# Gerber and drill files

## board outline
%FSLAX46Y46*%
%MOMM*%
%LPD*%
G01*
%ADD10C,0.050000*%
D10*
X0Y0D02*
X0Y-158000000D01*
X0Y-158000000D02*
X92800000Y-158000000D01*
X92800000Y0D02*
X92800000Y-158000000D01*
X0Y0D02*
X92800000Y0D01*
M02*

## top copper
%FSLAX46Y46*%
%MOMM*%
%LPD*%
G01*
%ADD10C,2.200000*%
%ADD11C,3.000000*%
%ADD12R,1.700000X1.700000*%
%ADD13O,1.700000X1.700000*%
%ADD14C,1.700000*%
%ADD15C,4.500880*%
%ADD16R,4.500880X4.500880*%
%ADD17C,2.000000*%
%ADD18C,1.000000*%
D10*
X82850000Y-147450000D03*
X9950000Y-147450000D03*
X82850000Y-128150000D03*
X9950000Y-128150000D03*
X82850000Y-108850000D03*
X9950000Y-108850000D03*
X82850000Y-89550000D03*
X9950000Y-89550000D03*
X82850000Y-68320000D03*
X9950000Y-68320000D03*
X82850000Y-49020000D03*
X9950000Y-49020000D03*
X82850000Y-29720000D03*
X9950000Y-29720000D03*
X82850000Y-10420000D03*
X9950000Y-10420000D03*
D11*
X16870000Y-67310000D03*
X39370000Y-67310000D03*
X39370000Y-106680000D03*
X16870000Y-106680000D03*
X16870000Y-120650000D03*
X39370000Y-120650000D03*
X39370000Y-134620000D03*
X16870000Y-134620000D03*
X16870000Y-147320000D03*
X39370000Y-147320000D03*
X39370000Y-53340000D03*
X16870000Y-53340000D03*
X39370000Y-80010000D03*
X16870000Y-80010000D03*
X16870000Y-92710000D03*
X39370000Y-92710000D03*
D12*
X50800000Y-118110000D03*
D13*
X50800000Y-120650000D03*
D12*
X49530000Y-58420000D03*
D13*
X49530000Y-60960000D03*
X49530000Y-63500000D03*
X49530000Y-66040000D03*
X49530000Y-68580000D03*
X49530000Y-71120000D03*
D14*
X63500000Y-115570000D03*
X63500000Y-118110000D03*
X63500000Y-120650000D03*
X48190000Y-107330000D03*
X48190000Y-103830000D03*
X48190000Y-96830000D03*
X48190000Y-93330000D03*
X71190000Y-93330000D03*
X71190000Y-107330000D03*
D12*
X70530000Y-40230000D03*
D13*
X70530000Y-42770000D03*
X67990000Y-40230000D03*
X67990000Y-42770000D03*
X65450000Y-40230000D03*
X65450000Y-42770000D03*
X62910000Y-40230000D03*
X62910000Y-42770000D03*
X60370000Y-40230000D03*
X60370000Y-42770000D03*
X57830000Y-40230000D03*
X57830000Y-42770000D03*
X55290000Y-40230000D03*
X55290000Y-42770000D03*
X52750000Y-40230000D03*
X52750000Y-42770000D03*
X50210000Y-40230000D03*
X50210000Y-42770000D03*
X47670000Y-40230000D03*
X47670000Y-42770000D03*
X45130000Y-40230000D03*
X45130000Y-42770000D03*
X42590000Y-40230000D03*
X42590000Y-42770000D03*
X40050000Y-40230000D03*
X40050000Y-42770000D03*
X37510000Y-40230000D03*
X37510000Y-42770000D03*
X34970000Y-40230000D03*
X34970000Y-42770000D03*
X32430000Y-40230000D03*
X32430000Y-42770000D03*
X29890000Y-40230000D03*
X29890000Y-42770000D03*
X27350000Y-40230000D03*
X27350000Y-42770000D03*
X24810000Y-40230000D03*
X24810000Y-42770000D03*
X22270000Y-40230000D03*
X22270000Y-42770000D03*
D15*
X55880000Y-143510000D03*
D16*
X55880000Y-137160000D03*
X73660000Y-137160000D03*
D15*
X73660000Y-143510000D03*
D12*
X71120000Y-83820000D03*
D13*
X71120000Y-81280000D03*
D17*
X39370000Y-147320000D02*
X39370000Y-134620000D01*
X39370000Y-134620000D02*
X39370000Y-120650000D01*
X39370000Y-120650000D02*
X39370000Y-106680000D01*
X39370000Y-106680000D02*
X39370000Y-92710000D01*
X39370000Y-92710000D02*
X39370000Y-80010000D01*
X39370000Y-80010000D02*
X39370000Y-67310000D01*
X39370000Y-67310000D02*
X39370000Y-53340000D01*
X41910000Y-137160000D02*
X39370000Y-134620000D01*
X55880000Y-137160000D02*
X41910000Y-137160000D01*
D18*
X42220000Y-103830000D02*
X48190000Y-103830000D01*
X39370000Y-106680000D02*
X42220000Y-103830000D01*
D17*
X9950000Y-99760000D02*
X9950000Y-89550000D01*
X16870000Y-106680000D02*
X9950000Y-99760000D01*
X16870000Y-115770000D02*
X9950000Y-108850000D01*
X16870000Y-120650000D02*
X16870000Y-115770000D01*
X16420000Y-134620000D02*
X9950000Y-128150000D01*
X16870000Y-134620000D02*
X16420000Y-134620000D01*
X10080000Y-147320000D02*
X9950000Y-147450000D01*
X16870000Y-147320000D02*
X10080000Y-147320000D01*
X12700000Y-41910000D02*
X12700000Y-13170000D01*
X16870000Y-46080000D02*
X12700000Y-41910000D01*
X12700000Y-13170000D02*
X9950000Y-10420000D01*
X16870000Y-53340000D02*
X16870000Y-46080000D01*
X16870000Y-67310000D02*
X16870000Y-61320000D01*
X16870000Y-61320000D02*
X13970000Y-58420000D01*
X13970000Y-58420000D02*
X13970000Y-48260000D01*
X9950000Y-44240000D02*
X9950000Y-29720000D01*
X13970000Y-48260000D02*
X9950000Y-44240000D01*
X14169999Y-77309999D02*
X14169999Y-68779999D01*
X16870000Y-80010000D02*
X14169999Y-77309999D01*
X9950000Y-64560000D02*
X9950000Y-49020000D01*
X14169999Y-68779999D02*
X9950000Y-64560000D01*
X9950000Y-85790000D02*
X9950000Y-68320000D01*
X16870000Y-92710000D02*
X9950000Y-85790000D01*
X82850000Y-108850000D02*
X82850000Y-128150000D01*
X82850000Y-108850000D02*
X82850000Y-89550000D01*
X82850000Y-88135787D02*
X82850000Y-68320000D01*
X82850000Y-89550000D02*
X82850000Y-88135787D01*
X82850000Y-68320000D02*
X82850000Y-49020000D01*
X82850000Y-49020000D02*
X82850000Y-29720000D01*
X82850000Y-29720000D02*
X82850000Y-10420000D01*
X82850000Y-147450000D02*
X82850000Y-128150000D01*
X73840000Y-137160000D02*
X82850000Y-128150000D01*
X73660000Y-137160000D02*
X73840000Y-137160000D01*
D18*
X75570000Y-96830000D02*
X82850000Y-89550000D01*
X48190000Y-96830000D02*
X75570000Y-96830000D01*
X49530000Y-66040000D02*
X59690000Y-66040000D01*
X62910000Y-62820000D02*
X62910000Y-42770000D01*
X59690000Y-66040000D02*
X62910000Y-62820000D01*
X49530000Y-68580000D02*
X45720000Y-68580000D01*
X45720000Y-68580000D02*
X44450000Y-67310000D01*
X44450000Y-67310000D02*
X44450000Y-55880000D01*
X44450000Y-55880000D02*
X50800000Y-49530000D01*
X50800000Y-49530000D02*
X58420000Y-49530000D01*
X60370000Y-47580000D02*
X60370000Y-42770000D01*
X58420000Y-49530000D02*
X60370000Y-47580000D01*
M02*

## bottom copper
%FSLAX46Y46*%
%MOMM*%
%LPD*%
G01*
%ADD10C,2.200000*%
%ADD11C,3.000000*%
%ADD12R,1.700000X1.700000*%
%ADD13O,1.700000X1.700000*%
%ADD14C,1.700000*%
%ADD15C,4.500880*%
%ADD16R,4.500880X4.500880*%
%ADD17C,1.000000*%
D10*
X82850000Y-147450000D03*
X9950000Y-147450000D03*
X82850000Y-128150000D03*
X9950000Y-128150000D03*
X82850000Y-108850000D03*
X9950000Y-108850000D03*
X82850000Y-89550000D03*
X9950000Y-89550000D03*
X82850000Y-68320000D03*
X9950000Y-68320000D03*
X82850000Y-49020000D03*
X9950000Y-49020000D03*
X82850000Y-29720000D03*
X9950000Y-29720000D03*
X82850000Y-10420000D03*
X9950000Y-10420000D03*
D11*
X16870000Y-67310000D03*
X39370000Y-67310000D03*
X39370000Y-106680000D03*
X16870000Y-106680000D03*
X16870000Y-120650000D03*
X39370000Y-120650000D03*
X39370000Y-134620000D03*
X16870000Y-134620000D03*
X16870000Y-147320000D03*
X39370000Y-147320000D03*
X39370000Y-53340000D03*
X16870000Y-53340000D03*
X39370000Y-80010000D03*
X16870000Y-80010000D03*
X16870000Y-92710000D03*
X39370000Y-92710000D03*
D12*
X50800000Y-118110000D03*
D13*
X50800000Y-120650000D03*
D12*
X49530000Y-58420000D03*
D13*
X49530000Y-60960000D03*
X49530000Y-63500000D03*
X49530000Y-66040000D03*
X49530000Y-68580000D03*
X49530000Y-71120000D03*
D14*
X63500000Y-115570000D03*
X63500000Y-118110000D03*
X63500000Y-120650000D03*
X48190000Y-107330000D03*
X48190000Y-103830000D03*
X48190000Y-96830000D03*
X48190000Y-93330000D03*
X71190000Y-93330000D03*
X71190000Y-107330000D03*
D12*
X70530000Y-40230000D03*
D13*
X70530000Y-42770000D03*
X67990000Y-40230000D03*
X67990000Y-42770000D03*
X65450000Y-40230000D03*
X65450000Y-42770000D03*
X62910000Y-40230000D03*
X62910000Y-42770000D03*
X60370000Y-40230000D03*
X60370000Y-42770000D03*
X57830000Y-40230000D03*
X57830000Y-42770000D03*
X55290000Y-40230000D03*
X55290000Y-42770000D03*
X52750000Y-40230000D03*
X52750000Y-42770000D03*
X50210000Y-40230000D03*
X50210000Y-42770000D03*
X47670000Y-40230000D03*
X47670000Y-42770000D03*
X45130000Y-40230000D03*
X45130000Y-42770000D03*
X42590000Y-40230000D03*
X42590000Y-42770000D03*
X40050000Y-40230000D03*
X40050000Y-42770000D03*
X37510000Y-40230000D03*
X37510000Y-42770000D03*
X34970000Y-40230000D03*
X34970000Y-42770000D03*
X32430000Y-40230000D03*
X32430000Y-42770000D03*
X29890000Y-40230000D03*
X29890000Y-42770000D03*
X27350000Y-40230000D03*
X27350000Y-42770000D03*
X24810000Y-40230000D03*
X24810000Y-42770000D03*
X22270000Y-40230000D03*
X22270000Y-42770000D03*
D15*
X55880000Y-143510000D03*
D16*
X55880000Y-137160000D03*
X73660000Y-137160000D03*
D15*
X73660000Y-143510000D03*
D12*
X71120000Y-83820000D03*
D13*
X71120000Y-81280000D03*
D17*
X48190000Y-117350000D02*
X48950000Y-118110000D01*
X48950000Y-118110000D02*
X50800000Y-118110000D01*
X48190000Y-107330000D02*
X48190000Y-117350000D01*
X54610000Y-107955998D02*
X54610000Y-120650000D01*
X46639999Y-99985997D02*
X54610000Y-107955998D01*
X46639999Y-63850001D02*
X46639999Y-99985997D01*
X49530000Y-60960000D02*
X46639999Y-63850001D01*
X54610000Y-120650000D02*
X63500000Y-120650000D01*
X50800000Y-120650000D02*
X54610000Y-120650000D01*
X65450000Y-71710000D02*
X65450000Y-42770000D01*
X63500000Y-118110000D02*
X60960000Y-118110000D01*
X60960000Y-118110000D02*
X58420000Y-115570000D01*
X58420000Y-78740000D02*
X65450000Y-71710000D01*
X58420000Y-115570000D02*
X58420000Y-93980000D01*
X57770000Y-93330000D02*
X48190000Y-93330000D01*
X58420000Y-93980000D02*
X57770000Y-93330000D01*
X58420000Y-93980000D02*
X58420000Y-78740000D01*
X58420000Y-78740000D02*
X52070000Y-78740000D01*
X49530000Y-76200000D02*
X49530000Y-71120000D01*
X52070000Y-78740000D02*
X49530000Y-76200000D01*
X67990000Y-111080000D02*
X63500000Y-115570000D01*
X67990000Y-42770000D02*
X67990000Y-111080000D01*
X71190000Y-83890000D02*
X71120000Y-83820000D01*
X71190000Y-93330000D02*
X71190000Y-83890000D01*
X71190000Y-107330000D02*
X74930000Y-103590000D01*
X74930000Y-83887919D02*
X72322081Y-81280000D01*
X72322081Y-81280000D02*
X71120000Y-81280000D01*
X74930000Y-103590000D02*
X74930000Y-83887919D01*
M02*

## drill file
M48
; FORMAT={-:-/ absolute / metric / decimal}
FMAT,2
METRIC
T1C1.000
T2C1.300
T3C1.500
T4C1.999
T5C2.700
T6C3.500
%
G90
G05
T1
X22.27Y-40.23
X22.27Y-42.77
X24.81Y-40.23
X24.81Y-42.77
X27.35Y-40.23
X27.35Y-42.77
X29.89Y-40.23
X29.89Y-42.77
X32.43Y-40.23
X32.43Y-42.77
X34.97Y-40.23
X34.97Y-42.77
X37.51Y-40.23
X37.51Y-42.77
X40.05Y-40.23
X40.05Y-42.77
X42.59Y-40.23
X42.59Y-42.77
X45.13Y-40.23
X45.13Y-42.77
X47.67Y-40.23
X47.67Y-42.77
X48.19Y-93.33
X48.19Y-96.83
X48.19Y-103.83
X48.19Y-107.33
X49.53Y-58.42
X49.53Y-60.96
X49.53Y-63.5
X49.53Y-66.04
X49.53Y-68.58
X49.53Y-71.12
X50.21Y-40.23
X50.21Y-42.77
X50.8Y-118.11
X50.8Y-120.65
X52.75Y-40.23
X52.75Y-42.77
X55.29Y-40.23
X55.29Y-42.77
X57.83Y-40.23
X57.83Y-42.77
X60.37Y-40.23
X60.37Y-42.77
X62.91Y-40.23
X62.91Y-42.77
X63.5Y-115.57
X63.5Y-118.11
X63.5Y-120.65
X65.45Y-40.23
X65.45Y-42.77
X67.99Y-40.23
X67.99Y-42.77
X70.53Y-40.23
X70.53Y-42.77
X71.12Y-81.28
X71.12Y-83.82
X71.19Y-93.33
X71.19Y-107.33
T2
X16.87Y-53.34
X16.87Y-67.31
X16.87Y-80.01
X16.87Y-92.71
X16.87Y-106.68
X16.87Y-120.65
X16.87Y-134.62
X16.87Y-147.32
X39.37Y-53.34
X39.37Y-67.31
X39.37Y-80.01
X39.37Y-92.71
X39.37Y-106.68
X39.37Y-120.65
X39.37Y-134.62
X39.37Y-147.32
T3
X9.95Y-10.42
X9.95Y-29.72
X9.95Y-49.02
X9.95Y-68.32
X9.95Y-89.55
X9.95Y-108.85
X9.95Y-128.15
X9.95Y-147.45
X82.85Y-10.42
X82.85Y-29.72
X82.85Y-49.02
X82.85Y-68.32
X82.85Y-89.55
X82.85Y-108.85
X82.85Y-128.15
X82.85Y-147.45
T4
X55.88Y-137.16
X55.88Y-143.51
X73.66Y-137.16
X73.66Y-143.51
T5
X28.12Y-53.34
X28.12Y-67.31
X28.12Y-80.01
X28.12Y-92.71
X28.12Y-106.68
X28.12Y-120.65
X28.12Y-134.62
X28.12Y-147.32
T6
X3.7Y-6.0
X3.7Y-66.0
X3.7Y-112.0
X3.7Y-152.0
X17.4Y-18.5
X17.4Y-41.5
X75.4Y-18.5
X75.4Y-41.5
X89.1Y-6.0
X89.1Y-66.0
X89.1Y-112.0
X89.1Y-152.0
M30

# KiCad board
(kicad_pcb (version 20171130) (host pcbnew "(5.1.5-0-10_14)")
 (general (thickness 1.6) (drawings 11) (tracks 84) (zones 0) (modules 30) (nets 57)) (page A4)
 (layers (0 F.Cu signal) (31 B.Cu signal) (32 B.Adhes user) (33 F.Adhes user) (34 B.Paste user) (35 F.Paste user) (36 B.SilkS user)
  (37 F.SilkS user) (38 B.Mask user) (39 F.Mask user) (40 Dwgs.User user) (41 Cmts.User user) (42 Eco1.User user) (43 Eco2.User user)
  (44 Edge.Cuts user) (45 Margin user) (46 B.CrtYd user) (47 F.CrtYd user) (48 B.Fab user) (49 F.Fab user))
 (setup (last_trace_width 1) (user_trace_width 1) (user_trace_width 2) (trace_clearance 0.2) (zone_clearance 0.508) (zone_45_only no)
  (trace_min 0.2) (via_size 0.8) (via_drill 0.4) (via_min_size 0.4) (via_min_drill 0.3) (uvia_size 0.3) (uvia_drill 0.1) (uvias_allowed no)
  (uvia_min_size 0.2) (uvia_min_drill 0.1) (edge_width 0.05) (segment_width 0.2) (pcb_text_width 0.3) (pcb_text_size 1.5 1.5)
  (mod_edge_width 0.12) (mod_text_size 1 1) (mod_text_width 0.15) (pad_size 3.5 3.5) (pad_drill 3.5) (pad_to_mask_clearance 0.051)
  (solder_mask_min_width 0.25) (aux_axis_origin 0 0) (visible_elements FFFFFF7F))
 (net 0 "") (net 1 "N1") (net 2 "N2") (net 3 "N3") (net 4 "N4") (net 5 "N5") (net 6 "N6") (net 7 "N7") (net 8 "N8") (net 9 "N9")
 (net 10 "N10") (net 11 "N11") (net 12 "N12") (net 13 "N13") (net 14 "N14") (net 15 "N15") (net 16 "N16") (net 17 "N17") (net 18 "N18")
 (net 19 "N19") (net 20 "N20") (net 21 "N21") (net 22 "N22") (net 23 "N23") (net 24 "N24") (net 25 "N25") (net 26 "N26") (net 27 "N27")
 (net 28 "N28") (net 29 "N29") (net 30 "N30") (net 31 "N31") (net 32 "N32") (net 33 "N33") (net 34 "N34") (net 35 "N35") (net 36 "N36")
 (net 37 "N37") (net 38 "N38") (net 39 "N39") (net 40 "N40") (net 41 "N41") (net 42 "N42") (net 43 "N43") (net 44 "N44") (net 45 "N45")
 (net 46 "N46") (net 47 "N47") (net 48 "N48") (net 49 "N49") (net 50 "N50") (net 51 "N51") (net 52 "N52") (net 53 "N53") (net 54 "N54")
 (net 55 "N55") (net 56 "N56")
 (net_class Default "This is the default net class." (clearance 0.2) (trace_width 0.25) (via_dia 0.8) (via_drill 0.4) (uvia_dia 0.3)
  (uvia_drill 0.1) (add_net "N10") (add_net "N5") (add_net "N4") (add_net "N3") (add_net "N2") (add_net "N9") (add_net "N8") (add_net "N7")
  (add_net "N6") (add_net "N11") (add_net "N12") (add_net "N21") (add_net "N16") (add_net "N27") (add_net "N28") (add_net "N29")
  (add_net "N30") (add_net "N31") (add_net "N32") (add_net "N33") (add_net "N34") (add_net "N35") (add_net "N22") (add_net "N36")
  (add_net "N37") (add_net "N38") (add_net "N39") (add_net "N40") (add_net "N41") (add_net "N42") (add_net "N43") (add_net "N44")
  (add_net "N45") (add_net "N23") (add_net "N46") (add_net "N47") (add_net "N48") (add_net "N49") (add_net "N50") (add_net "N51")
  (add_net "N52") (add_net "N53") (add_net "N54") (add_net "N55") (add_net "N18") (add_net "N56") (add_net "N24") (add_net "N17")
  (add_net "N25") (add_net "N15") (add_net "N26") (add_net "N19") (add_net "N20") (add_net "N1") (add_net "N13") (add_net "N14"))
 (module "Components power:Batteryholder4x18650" (layer F.Cu) (at 46.4 118.5)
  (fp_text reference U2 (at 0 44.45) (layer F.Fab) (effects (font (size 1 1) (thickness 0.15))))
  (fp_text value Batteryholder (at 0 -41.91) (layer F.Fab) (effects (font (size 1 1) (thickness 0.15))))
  (pad 8 thru_hole circle (at 36.45 28.95) (size 2.2 2.2) (drill 1.5) (layers *.Cu *.Mask) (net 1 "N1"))
  (pad 7 thru_hole circle (at -36.45 28.95) (size 2.2 2.2) (drill 1.5) (layers *.Cu *.Mask) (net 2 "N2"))
  (pad 6 thru_hole circle (at 36.45 9.65) (size 2.2 2.2) (drill 1.5) (layers *.Cu *.Mask) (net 1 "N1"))
  (pad 5 thru_hole circle (at -36.45 9.65) (size 2.2 2.2) (drill 1.5) (layers *.Cu *.Mask) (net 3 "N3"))
  (pad 4 thru_hole circle (at 36.45 -9.65) (size 2.2 2.2) (drill 1.5) (layers *.Cu *.Mask) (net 1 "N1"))
  (pad 3 thru_hole circle (at -36.45 -9.65) (size 2.2 2.2) (drill 1.5) (layers *.Cu *.Mask) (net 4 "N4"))
  (pad 2 thru_hole circle (at 36.45 -28.95) (size 2.2 2.2) (drill 1.5) (layers *.Cu *.Mask) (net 1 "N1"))
  (pad 1 thru_hole circle (at -36.45 -28.95) (size 2.2 2.2) (drill 1.5) (layers *.Cu *.Mask) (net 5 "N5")))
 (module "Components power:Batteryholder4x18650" (layer F.Cu) (at 46.4 39.37)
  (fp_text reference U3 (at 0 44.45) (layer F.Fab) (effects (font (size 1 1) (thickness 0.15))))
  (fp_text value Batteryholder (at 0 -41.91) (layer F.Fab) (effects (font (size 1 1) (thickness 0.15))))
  (pad 8 thru_hole circle (at 36.45 28.95) (size 2.2 2.2) (drill 1.5) (layers *.Cu *.Mask) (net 1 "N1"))
  (pad 7 thru_hole circle (at -36.45 28.95) (size 2.2 2.2) (drill 1.5) (layers *.Cu *.Mask) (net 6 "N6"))
  (pad 6 thru_hole circle (at 36.45 9.65) (size 2.2 2.2) (drill 1.5) (layers *.Cu *.Mask) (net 1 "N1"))
  (pad 5 thru_hole circle (at -36.45 9.65) (size 2.2 2.2) (drill 1.5) (layers *.Cu *.Mask) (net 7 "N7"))
  (pad 4 thru_hole circle (at 36.45 -9.65) (size 2.2 2.2) (drill 1.5) (layers *.Cu *.Mask) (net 1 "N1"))
  (pad 3 thru_hole circle (at -36.45 -9.65) (size 2.2 2.2) (drill 1.5) (layers *.Cu *.Mask) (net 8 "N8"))
  (pad 2 thru_hole circle (at 36.45 -28.95) (size 2.2 2.2) (drill 1.5) (layers *.Cu *.Mask) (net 1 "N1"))
  (pad 1 thru_hole circle (at -36.45 -28.95) (size 2.2 2.2) (drill 1.5) (layers *.Cu *.Mask) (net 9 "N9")))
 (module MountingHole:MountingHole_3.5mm (layer F.Cu) (at 3.7 112)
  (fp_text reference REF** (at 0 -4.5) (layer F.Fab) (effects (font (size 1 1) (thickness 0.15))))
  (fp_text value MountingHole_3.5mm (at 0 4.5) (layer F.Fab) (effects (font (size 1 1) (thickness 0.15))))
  (pad 1 np_thru_hole circle (at 0 0) (size 3.5 3.5) (drill 3.5) (layers *.Cu *.Mask)))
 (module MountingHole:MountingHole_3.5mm (layer F.Cu) (at 89.1 66)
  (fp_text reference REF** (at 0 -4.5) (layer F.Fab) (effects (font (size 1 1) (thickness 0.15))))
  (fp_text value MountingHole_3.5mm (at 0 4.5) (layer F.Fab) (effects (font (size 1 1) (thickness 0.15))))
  (pad 1 np_thru_hole circle (at 0 0) (size 3.5 3.5) (drill 3.5) (layers *.Cu *.Mask)))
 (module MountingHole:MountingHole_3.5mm (layer F.Cu) (at 3.7 66)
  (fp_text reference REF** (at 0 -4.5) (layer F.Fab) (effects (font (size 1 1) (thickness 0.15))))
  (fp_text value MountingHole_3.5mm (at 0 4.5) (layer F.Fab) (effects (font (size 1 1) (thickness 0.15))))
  (pad 1 np_thru_hole circle (at 0 0) (size 3.5 3.5) (drill 3.5) (layers *.Cu *.Mask)))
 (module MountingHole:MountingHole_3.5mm (layer F.Cu) (at 89.1 112)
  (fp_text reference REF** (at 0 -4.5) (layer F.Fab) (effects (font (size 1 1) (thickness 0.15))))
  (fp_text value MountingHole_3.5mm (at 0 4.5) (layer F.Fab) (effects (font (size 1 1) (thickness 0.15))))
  (pad 1 np_thru_hole circle (at 0 0) (size 3.5 3.5) (drill 3.5) (layers *.Cu *.Mask)))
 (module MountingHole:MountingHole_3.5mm (layer F.Cu) (at 89.1 6)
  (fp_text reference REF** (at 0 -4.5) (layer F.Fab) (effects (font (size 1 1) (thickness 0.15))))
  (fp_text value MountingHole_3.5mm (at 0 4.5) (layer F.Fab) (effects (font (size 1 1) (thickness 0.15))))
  (pad 1 np_thru_hole circle (at 0 0) (size 3.5 3.5) (drill 3.5) (layers *.Cu *.Mask)))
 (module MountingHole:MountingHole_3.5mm (layer F.Cu) (at 89.1 152)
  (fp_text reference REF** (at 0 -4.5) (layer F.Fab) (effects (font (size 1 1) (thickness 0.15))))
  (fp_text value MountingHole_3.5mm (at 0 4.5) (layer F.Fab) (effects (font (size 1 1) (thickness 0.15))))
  (pad 1 np_thru_hole circle (at 0 0) (size 3.5 3.5) (drill 3.5) (layers *.Cu *.Mask)))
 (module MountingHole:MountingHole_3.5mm (layer F.Cu) (at 3.7 6)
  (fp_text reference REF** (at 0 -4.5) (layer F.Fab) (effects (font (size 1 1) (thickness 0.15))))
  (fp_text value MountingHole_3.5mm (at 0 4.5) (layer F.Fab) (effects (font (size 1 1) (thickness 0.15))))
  (pad 1 np_thru_hole circle (at 0 0) (size 3.5 3.5) (drill 3.5) (layers *.Cu *.Mask)))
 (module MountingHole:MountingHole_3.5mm (layer F.Cu) (at 3.7 152)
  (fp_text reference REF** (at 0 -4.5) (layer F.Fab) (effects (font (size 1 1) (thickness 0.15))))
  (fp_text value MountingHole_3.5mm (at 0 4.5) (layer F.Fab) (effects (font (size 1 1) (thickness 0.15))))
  (pad 1 np_thru_hole circle (at 0 0) (size 3.5 3.5) (drill 3.5) (layers *.Cu *.Mask)))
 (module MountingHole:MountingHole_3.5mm (layer F.Cu) (at 75.4 41.5)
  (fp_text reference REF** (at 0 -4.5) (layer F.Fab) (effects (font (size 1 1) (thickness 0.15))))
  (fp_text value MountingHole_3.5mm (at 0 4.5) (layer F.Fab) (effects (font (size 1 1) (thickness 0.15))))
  (pad 1 np_thru_hole circle (at 0 0) (size 3.5 3.5) (drill 3.5) (layers *.Cu *.Mask)))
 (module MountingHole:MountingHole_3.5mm (layer F.Cu) (at 75.4 18.5)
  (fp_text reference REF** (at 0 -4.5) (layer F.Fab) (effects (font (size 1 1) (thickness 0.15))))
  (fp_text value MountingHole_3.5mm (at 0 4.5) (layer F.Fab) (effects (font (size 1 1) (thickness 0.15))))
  (pad 1 np_thru_hole circle (at 0 0) (size 3.5 3.5) (drill 3.5) (layers *.Cu *.Mask)))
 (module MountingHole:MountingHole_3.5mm (layer F.Cu) (at 17.4 18.5)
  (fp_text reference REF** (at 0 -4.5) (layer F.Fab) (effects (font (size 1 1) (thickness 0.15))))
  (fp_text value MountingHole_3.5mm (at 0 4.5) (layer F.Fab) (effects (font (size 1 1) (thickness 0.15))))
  (pad 1 np_thru_hole circle (at 0 0) (size 3.5 3.5) (drill 3.5) (layers *.Cu *.Mask)))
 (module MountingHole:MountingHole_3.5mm (layer F.Cu) (at 17.4 41.5)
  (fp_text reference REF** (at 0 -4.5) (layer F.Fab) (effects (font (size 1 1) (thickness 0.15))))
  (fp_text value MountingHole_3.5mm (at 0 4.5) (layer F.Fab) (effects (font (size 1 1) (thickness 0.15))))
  (pad 1 np_thru_hole circle (at 0 0) (size 3.5 3.5) (drill 3.5) (layers *.Cu *.Mask)))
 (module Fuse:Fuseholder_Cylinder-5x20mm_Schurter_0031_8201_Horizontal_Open (layer F.Cu) (at 39.37 67.31 180)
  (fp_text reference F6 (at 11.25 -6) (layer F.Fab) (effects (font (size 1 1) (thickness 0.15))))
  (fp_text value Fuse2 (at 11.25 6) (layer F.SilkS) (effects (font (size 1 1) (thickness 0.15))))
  (pad "" np_thru_hole circle (at 11.25 0 180) (size 2.7 2.7) (drill 2.7) (layers *.Cu *.Mask))
  (pad 2 thru_hole circle (at 22.5 0 180) (size 3 3) (drill 1.3) (layers *.Cu *.Mask) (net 8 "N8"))
  (pad 1 thru_hole circle (at 0 0 180) (size 3 3) (drill 1.3) (layers *.Cu *.Mask) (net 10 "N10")))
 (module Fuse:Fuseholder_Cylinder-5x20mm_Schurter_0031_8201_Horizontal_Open (layer F.Cu) (at 39.37 106.68 180)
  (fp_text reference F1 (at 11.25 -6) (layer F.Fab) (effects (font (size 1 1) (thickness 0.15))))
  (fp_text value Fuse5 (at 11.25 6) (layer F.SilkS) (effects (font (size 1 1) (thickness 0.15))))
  (pad 1 thru_hole circle (at 0 0 180) (size 3 3) (drill 1.3) (layers *.Cu *.Mask) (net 10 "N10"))
  (pad 2 thru_hole circle (at 22.5 0 180) (size 3 3) (drill 1.3) (layers *.Cu *.Mask) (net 5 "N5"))
  (pad "" np_thru_hole circle (at 11.25 0 180) (size 2.7 2.7) (drill 2.7) (layers *.Cu *.Mask)))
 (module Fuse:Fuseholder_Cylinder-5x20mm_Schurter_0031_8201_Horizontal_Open (layer F.Cu) (at 39.37 120.65 180)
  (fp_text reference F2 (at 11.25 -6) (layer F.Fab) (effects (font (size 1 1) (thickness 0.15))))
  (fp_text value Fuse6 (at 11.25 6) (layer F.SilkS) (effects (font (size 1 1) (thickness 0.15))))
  (pad "" np_thru_hole circle (at 11.25 0 180) (size 2.7 2.7) (drill 2.7) (layers *.Cu *.Mask))
  (pad 2 thru_hole circle (at 22.5 0 180) (size 3 3) (drill 1.3) (layers *.Cu *.Mask) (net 4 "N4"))
  (pad 1 thru_hole circle (at 0 0 180) (size 3 3) (drill 1.3) (layers *.Cu *.Mask) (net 10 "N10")))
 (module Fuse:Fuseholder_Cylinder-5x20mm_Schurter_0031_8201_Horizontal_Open (layer F.Cu) (at 39.37 134.62 180)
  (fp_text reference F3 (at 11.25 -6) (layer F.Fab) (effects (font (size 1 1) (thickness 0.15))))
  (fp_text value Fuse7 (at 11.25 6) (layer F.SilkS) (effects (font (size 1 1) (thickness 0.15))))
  (pad 1 thru_hole circle (at 0 0 180) (size 3 3) (drill 1.3) (layers *.Cu *.Mask) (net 10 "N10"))
  (pad 2 thru_hole circle (at 22.5 0 180) (size 3 3) (drill 1.3) (layers *.Cu *.Mask) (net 3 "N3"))
  (pad "" np_thru_hole circle (at 11.25 0 180) (size 2.7 2.7) (drill 2.7) (layers *.Cu *.Mask)))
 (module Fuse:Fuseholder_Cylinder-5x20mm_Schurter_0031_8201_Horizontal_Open (layer F.Cu) (at 39.37 147.32 180)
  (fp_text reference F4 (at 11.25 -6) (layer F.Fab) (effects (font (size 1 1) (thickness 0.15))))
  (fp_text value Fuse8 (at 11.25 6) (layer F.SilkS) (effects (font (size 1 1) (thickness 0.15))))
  (pad "" np_thru_hole circle (at 11.25 0 180) (size 2.7 2.7) (drill 2.7) (layers *.Cu *.Mask))
  (pad 2 thru_hole circle (at 22.5 0 180) (size 3 3) (drill 1.3) (layers *.Cu *.Mask) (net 2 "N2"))
  (pad 1 thru_hole circle (at 0 0 180) (size 3 3) (drill 1.3) (layers *.Cu *.Mask) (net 10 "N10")))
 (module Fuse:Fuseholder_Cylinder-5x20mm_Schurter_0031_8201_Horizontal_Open (layer F.Cu) (at 39.37 53.34 180)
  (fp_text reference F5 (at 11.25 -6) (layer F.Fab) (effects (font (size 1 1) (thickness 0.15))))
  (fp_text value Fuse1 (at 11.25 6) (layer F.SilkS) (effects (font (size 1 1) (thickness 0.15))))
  (pad 1 thru_hole circle (at 0 0 180) (size 3 3) (drill 1.3) (layers *.Cu *.Mask) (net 10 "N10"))
  (pad 2 thru_hole circle (at 22.5 0 180) (size 3 3) (drill 1.3) (layers *.Cu *.Mask) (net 9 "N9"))
  (pad "" np_thru_hole circle (at 11.25 0 180) (size 2.7 2.7) (drill 2.7) (layers *.Cu *.Mask)))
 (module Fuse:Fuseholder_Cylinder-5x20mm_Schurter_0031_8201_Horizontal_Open (layer F.Cu) (at 39.37 80.01 180)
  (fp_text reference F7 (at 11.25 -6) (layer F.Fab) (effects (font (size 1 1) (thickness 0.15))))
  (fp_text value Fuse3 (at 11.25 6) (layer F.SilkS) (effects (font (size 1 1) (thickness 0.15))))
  (pad 1 thru_hole circle (at 0 0 180) (size 3 3) (drill 1.3) (layers *.Cu *.Mask) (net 10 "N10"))
  (pad 2 thru_hole circle (at 22.5 0 180) (size 3 3) (drill 1.3) (layers *.Cu *.Mask) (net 7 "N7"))
  (pad "" np_thru_hole circle (at 11.25 0 180) (size 2.7 2.7) (drill 2.7) (layers *.Cu *.Mask)))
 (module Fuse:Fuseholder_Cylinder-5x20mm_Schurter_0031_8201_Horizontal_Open (layer F.Cu) (at 39.37 92.71 180)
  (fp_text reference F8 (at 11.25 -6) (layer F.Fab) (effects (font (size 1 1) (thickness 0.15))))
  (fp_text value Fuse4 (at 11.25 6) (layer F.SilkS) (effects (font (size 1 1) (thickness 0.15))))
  (pad "" np_thru_hole circle (at 11.25 0 180) (size 2.7 2.7) (drill 2.7) (layers *.Cu *.Mask))
  (pad 2 thru_hole circle (at 22.5 0 180) (size 3 3) (drill 1.3) (layers *.Cu *.Mask) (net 6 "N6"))
  (pad 1 thru_hole circle (at 0 0 180) (size 3 3) (drill 1.3) (layers *.Cu *.Mask) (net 10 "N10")))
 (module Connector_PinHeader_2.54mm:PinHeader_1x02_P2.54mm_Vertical (layer F.Cu) (at 50.8 118.11)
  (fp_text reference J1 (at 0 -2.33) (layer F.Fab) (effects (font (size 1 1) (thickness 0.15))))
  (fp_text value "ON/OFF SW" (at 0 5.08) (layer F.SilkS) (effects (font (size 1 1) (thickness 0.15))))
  (pad 1 thru_hole rect (at 0 0) (size 1.7 1.7) (drill 1) (layers *.Cu *.Mask) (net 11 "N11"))
  (pad 2 thru_hole oval (at 0 2.54) (size 1.7 1.7) (drill 1) (layers *.Cu *.Mask) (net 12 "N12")))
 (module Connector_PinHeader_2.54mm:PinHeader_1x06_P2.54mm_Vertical (layer F.Cu) (at 49.53 58.42)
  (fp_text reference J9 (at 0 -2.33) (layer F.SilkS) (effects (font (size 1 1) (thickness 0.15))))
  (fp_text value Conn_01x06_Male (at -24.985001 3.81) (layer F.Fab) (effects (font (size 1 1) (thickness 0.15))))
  (pad 1 thru_hole rect (at 0 0) (size 1.7 1.7) (drill 1) (layers *.Cu *.Mask) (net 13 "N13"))
  (pad 2 thru_hole oval (at 0 2.54) (size 1.7 1.7) (drill 1) (layers *.Cu *.Mask) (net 12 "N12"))
  (pad 3 thru_hole oval (at 0 5.08) (size 1.7 1.7) (drill 1) (layers *.Cu *.Mask) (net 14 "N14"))
  (pad 4 thru_hole oval (at 0 7.62) (size 1.7 1.7) (drill 1) (layers *.Cu *.Mask) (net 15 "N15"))
  (pad 5 thru_hole oval (at 0 10.16) (size 1.7 1.7) (drill 1) (layers *.Cu *.Mask) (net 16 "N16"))
  (pad 6 thru_hole oval (at 0 12.7) (size 1.7 1.7) (drill 1) (layers *.Cu *.Mask) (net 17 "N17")))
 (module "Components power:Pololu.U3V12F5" (layer F.Cu) (at 68.58 118.11 270)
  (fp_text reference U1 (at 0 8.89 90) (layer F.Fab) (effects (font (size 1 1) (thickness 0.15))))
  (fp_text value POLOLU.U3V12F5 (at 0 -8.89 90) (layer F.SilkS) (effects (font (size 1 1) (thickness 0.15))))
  (pad 3 thru_hole circle (at -2.54 5.08 270) (size 1.7 1.7) (drill 1) (layers *.Cu *.Mask) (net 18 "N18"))
  (pad 2 thru_hole circle (at 0 5.08 270) (size 1.7 1.7) (drill 1) (layers *.Cu *.Mask) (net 17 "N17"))
  (pad 1 thru_hole circle (at 2.54 5.08 270) (size 1.7 1.7) (drill 1) (layers *.Cu *.Mask) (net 12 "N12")))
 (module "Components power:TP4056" (layer F.Cu) (at 59.69 100.33 90)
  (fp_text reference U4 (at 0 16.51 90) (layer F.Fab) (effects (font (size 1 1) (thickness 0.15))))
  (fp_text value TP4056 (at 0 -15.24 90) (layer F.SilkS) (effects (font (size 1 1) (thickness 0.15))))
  (pad 1 thru_hole circle (at -7 -11.5 90) (size 1.7 1.7) (drill 1) (layers *.Cu *.Mask) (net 11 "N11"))
  (pad 2 thru_hole circle (at -3.5 -11.5 90) (size 1.7 1.7) (drill 1) (layers *.Cu *.Mask) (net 10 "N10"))
  (pad 3 thru_hole circle (at 3.5 -11.5 90) (size 1.7 1.7) (drill 1) (layers *.Cu *.Mask) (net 1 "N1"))
  (pad 4 thru_hole circle (at 7 -11.5 90) (size 1.7 1.7) (drill 1) (layers *.Cu *.Mask) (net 17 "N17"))
  (pad 5 thru_hole circle (at 7 11.5 90) (size 1.7 1.7) (drill 1) (layers *.Cu *.Mask) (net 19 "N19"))
  (pad 6 thru_hole circle (at -7 11.5 90) (size 1.7 1.7) (drill 1) (layers *.Cu *.Mask) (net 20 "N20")))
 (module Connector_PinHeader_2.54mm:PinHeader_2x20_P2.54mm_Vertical (layer F.Cu) (at 70.53 40.23 270)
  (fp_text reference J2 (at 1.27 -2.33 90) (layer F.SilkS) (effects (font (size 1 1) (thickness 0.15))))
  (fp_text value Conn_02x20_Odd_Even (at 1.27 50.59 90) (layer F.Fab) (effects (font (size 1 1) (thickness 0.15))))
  (pad 1 thru_hole rect (at 0 0 270) (size 1.7 1.7) (drill 1) (layers *.Cu *.Mask) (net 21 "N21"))
  (pad 2 thru_hole oval (at 2.54 0 270) (size 1.7 1.7) (drill 1) (layers *.Cu *.Mask) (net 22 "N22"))
  (pad 3 thru_hole oval (at 0 2.54 270) (size 1.7 1.7) (drill 1) (layers *.Cu *.Mask) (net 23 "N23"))
  (pad 4 thru_hole oval (at 2.54 2.54 270) (size 1.7 1.7) (drill 1) (layers *.Cu *.Mask) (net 18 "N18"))
  (pad 5 thru_hole oval (at 0 5.08 270) (size 1.7 1.7) (drill 1) (layers *.Cu *.Mask) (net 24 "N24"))
  (pad 6 thru_hole oval (at 2.54 5.08 270) (size 1.7 1.7) (drill 1) (layers *.Cu *.Mask) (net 17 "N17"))
  (pad 7 thru_hole oval (at 0 7.62 270) (size 1.7 1.7) (drill 1) (layers *.Cu *.Mask) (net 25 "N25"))
  (pad 8 thru_hole oval (at 2.54 7.62 270) (size 1.7 1.7) (drill 1) (layers *.Cu *.Mask) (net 15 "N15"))
  (pad 9 thru_hole oval (at 0 10.16 270) (size 1.7 1.7) (drill 1) (layers *.Cu *.Mask) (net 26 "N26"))
  (pad 10 thru_hole oval (at 2.54 10.16 270) (size 1.7 1.7) (drill 1) (layers *.Cu *.Mask) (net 16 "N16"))
  (pad 11 thru_hole oval (at 0 12.7 270) (size 1.7 1.7) (drill 1) (layers *.Cu *.Mask) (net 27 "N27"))
  (pad 12 thru_hole oval (at 2.54 12.7 270) (size 1.7 1.7) (drill 1) (layers *.Cu *.Mask) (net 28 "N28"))
  (pad 13 thru_hole oval (at 0 15.24 270) (size 1.7 1.7) (drill 1) (layers *.Cu *.Mask) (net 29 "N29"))
  (pad 14 thru_hole oval (at 2.54 15.24 270) (size 1.7 1.7) (drill 1) (layers *.Cu *.Mask) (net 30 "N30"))
  (pad 15 thru_hole oval (at 0 17.78 270) (size 1.7 1.7) (drill 1) (layers *.Cu *.Mask) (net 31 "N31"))
  (pad 16 thru_hole oval (at 2.54 17.78 270) (size 1.7 1.7) (drill 1) (layers *.Cu *.Mask) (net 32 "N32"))
  (pad 17 thru_hole oval (at 0 20.32 270) (size 1.7 1.7) (drill 1) (layers *.Cu *.Mask) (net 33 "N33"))
  (pad 18 thru_hole oval (at 2.54 20.32 270) (size 1.7 1.7) (drill 1) (layers *.Cu *.Mask) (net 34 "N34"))
  (pad 19 thru_hole oval (at 0 22.86 270) (size 1.7 1.7) (drill 1) (layers *.Cu *.Mask) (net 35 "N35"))
  (pad 20 thru_hole oval (at 2.54 22.86 270) (size 1.7 1.7) (drill 1) (layers *.Cu *.Mask) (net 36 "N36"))
  (pad 21 thru_hole oval (at 0 25.4 270) (size 1.7 1.7) (drill 1) (layers *.Cu *.Mask) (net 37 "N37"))
  (pad 22 thru_hole oval (at 2.54 25.4 270) (size 1.7 1.7) (drill 1) (layers *.Cu *.Mask) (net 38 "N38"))
  (pad 23 thru_hole oval (at 0 27.94 270) (size 1.7 1.7) (drill 1) (layers *.Cu *.Mask) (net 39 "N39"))
  (pad 24 thru_hole oval (at 2.54 27.94 270) (size 1.7 1.7) (drill 1) (layers *.Cu *.Mask) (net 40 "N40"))
  (pad 25 thru_hole oval (at 0 30.48 270) (size 1.7 1.7) (drill 1) (layers *.Cu *.Mask) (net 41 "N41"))
  (pad 26 thru_hole oval (at 2.54 30.48 270) (size 1.7 1.7) (drill 1) (layers *.Cu *.Mask) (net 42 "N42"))
  (pad 27 thru_hole oval (at 0 33.02 270) (size 1.7 1.7) (drill 1) (layers *.Cu *.Mask) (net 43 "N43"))
  (pad 28 thru_hole oval (at 2.54 33.02 270) (size 1.7 1.7) (drill 1) (layers *.Cu *.Mask) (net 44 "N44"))
  (pad 29 thru_hole oval (at 0 35.56 270) (size 1.7 1.7) (drill 1) (layers *.Cu *.Mask) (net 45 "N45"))
  (pad 30 thru_hole oval (at 2.54 35.56 270) (size 1.7 1.7) (drill 1) (layers *.Cu *.Mask) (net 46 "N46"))
  (pad 31 thru_hole oval (at 0 38.1 270) (size 1.7 1.7) (drill 1) (layers *.Cu *.Mask) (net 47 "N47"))
  (pad 32 thru_hole oval (at 2.54 38.1 270) (size 1.7 1.7) (drill 1) (layers *.Cu *.Mask) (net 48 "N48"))
  (pad 33 thru_hole oval (at 0 40.64 270) (size 1.7 1.7) (drill 1) (layers *.Cu *.Mask) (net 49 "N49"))
  (pad 34 thru_hole oval (at 2.54 40.64 270) (size 1.7 1.7) (drill 1) (layers *.Cu *.Mask) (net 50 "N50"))
  (pad 35 thru_hole oval (at 0 43.18 270) (size 1.7 1.7) (drill 1) (layers *.Cu *.Mask) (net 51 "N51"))
  (pad 36 thru_hole oval (at 2.54 43.18 270) (size 1.7 1.7) (drill 1) (layers *.Cu *.Mask) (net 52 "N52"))
  (pad 37 thru_hole oval (at 0 45.72 270) (size 1.7 1.7) (drill 1) (layers *.Cu *.Mask) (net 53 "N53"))
  (pad 38 thru_hole oval (at 2.54 45.72 270) (size 1.7 1.7) (drill 1) (layers *.Cu *.Mask) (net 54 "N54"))
  (pad 39 thru_hole oval (at 0 48.26 270) (size 1.7 1.7) (drill 1) (layers *.Cu *.Mask) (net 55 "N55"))
  (pad 40 thru_hole oval (at 2.54 48.26 270) (size 1.7 1.7) (drill 1) (layers *.Cu *.Mask) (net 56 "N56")))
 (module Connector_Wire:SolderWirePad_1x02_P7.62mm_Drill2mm (layer F.Cu) (at 55.88 137.16 270)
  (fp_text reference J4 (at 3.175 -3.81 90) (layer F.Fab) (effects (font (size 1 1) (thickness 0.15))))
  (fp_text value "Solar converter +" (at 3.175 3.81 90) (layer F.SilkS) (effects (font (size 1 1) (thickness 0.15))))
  (pad 2 thru_hole circle (at 6.35 0 270) (size 4.50088 4.50088) (drill 1.99898) (layers *.Cu *.Mask))
  (pad 1 thru_hole rect (at 0 0 270) (size 4.50088 4.50088) (drill 1.99898) (layers *.Cu *.Mask) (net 10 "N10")))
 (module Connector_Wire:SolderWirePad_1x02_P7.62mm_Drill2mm (layer F.Cu) (at 73.66 137.16 270)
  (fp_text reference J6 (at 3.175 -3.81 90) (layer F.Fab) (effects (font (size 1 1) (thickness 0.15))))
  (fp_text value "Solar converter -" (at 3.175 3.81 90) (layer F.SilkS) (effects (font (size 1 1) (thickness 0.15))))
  (pad 1 thru_hole rect (at 0 0 270) (size 4.50088 4.50088) (drill 1.99898) (layers *.Cu *.Mask) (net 1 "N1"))
  (pad 2 thru_hole circle (at 6.35 0 270) (size 4.50088 4.50088) (drill 1.99898) (layers *.Cu *.Mask)))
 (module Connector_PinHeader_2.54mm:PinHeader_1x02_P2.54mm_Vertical (layer F.Cu) (at 71.12 83.82 180)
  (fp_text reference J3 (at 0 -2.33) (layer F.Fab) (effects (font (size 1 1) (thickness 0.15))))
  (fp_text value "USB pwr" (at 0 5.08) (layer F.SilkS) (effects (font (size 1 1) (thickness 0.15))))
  (pad 1 thru_hole rect (at 0 0 180) (size 1.7 1.7) (drill 1) (layers *.Cu *.Mask) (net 19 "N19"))
  (pad 2 thru_hole oval (at 0 2.54 180) (size 1.7 1.7) (drill 1) (layers *.Cu *.Mask) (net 20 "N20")))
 (gr_line (start 0 0) (end 0 158) (layer Edge.Cuts) (width 0.05))
 (gr_line (start 0 158) (end 92.8 158) (layer Edge.Cuts) (width 0.05))
 (gr_line (start 92.8 0) (end 92.8 158) (layer Edge.Cuts) (width 0.05))
 (gr_line (start 0 0) (end 92.8 0) (layer Edge.Cuts) (width 0.05))
 (segment (start 39.37 147.32) (end 39.37 134.62) (width 2) (layer F.Cu) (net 10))
 (segment (start 39.37 134.62) (end 39.37 120.65) (width 2) (layer F.Cu) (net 10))
 (segment (start 39.37 120.65) (end 39.37 106.68) (width 2) (layer F.Cu) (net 10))
 (segment (start 39.37 106.68) (end 39.37 92.71) (width 2) (layer F.Cu) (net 10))
 (segment (start 39.37 92.71) (end 39.37 80.01) (width 2) (layer F.Cu) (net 10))
 (segment (start 39.37 80.01) (end 39.37 67.31) (width 2) (layer F.Cu) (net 10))
 (segment (start 39.37 67.31) (end 39.37 53.34) (width 2) (layer F.Cu) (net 10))
 (segment (start 41.91 137.16) (end 39.37 134.62) (width 2) (layer F.Cu) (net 10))
 (segment (start 55.88 137.16) (end 41.91 137.16) (width 2) (layer F.Cu) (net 10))
 (segment (start 42.22 103.83) (end 48.19 103.83) (width 1) (layer F.Cu) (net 10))
 (segment (start 39.37 106.68) (end 42.22 103.83) (width 1) (layer F.Cu) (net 10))
 (segment (start 9.95 99.76) (end 9.95 89.55) (width 2) (layer F.Cu) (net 5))
 (segment (start 16.87 106.68) (end 9.95 99.76) (width 2) (layer F.Cu) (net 5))
 (segment (start 16.87 115.77) (end 9.95 108.85) (width 2) (layer F.Cu) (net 4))
 (segment (start 16.87 120.65) (end 16.87 115.77) (width 2) (layer F.Cu) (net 4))
 (segment (start 16.42 134.62) (end 9.95 128.15) (width 2) (layer F.Cu) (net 3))
 (segment (start 16.87 134.62) (end 16.42 134.62) (width 2) (layer F.Cu) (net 3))
 (segment (start 10.08 147.32) (end 9.95 147.45) (width 2) (layer F.Cu) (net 2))
 (segment (start 16.87 147.32) (end 10.08 147.32) (width 2) (layer F.Cu) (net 2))
 (segment (start 12.7 41.91) (end 12.7 13.17) (width 2) (layer F.Cu) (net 9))
 (segment (start 16.87 46.08) (end 12.7 41.91) (width 2) (layer F.Cu) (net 9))
 (segment (start 12.7 13.17) (end 9.95 10.42) (width 2) (layer F.Cu) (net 9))
 (segment (start 16.87 53.34) (end 16.87 46.08) (width 2) (layer F.Cu) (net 9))
 (segment (start 16.87 67.31) (end 16.87 61.32) (width 2) (layer F.Cu) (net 8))
 (segment (start 16.87 61.32) (end 13.97 58.42) (width 2) (layer F.Cu) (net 8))
 (segment (start 13.97 58.42) (end 13.97 48.26) (width 2) (layer F.Cu) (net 8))
 (segment (start 9.95 44.24) (end 9.95 29.72) (width 2) (layer F.Cu) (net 8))
 (segment (start 13.97 48.26) (end 9.95 44.24) (width 2) (layer F.Cu) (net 8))
 (segment (start 14.169999 77.309999) (end 14.169999 68.779999) (width 2) (layer F.Cu) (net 7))
 (segment (start 16.87 80.01) (end 14.169999 77.309999) (width 2) (layer F.Cu) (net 7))
 (segment (start 9.95 64.56) (end 9.95 49.02) (width 2) (layer F.Cu) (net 7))
 (segment (start 14.169999 68.779999) (end 9.95 64.56) (width 2) (layer F.Cu) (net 7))
 (segment (start 9.95 85.79) (end 9.95 68.32) (width 2) (layer F.Cu) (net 6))
 (segment (start 16.87 92.71) (end 9.95 85.79) (width 2) (layer F.Cu) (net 6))
 (segment (start 48.19 117.35) (end 48.95 118.11) (width 1) (layer B.Cu) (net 11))
 (segment (start 48.95 118.11) (end 50.8 118.11) (width 1) (layer B.Cu) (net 11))
 (segment (start 48.19 107.33) (end 48.19 117.35) (width 1) (layer B.Cu) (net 11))
 (segment (start 54.61 107.955998) (end 54.61 120.65) (width 1) (layer B.Cu) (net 12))
 (segment (start 46.639999 99.985997) (end 54.61 107.955998) (width 1) (layer B.Cu) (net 12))
 (segment (start 46.639999 63.850001) (end 46.639999 99.985997) (width 1) (layer B.Cu) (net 12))
 (segment (start 49.53 60.96) (end 46.639999 63.850001) (width 1) (layer B.Cu) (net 12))
 (segment (start 54.61 120.65) (end 63.5 120.65) (width 1) (layer B.Cu) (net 12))
 (segment (start 50.8 120.65) (end 54.61 120.65) (width 1) (layer B.Cu) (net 12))
 (segment (start 82.85 108.85) (end 82.85 128.15) (width 2) (layer F.Cu) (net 1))
 (segment (start 82.85 108.85) (end 82.85 89.55) (width 2) (layer F.Cu) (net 1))
 (segment (start 82.85 88.135787) (end 82.85 68.32) (width 2) (layer F.Cu) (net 1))
 (segment (start 82.85 89.55) (end 82.85 88.135787) (width 2) (layer F.Cu) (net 1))
 (segment (start 82.85 68.32) (end 82.85 49.02) (width 2) (layer F.Cu) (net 1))
 (segment (start 82.85 49.02) (end 82.85 29.72) (width 2) (layer F.Cu) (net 1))
 (segment (start 82.85 29.72) (end 82.85 10.42) (width 2) (layer F.Cu) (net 1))
 (segment (start 82.85 147.45) (end 82.85 128.15) (width 2) (layer F.Cu) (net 1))
 (segment (start 73.84 137.16) (end 82.85 128.15) (width 2) (layer F.Cu) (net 1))
 (segment (start 73.66 137.16) (end 73.84 137.16) (width 2) (layer F.Cu) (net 1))
 (segment (start 75.57 96.83) (end 82.85 89.55) (width 1) (layer F.Cu) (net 1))
 (segment (start 48.19 96.83) (end 75.57 96.83) (width 1) (layer F.Cu) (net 1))
 (segment (start 49.53 66.04) (end 59.69 66.04) (width 1) (layer F.Cu) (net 15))
 (segment (start 62.91 62.82) (end 62.91 42.77) (width 1) (layer F.Cu) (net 15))
 (segment (start 59.69 66.04) (end 62.91 62.82) (width 1) (layer F.Cu) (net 15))
 (segment (start 49.53 68.58) (end 45.72 68.58) (width 1) (layer F.Cu) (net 16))
 (segment (start 45.72 68.58) (end 44.45 67.31) (width 1) (layer F.Cu) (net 16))
 (segment (start 44.45 67.31) (end 44.45 55.88) (width 1) (layer F.Cu) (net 16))
 (segment (start 44.45 55.88) (end 50.8 49.53) (width 1) (layer F.Cu) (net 16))
 (segment (start 50.8 49.53) (end 58.42 49.53) (width 1) (layer F.Cu) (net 16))
 (segment (start 60.37 47.58) (end 60.37 42.77) (width 1) (layer F.Cu) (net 16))
 (segment (start 58.42 49.53) (end 60.37 47.58) (width 1) (layer F.Cu) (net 16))
 (segment (start 65.45 71.71) (end 65.45 42.77) (width 1) (layer B.Cu) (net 17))
 (segment (start 63.5 118.11) (end 60.96 118.11) (width 1) (layer B.Cu) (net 17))
 (segment (start 60.96 118.11) (end 58.42 115.57) (width 1) (layer B.Cu) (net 17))
 (segment (start 58.42 78.74) (end 65.45 71.71) (width 1) (layer B.Cu) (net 17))
 (segment (start 58.42 115.57) (end 58.42 93.98) (width 1) (layer B.Cu) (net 17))
 (segment (start 57.77 93.33) (end 48.19 93.33) (width 1) (layer B.Cu) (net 17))
 (segment (start 58.42 93.98) (end 57.77 93.33) (width 1) (layer B.Cu) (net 17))
 (segment (start 58.42 93.98) (end 58.42 78.74) (width 1) (layer B.Cu) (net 17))
 (segment (start 58.42 78.74) (end 52.07 78.74) (width 1) (layer B.Cu) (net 17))
 (segment (start 49.53 76.2) (end 49.53 71.12) (width 1) (layer B.Cu) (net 17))
 (segment (start 52.07 78.74) (end 49.53 76.2) (width 1) (layer B.Cu) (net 17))
 (segment (start 67.99 111.08) (end 63.5 115.57) (width 1) (layer B.Cu) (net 18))
 (segment (start 67.99 42.77) (end 67.99 111.08) (width 1) (layer B.Cu) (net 18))
 (segment (start 71.19 83.89) (end 71.12 83.82) (width 1) (layer B.Cu) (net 19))
 (segment (start 71.19 93.33) (end 71.19 83.89) (width 1) (layer B.Cu) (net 19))
 (segment (start 71.19 107.33) (end 74.93 103.59) (width 1) (layer B.Cu) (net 20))
 (segment (start 74.93 83.887919) (end 72.322081 81.28) (width 1) (layer B.Cu) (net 20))
 (segment (start 72.322081 81.28) (end 71.12 81.28) (width 1) (layer B.Cu) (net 20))
 (segment (start 74.93 103.59) (end 74.93 83.887919) (width 1) (layer B.Cu) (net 20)))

